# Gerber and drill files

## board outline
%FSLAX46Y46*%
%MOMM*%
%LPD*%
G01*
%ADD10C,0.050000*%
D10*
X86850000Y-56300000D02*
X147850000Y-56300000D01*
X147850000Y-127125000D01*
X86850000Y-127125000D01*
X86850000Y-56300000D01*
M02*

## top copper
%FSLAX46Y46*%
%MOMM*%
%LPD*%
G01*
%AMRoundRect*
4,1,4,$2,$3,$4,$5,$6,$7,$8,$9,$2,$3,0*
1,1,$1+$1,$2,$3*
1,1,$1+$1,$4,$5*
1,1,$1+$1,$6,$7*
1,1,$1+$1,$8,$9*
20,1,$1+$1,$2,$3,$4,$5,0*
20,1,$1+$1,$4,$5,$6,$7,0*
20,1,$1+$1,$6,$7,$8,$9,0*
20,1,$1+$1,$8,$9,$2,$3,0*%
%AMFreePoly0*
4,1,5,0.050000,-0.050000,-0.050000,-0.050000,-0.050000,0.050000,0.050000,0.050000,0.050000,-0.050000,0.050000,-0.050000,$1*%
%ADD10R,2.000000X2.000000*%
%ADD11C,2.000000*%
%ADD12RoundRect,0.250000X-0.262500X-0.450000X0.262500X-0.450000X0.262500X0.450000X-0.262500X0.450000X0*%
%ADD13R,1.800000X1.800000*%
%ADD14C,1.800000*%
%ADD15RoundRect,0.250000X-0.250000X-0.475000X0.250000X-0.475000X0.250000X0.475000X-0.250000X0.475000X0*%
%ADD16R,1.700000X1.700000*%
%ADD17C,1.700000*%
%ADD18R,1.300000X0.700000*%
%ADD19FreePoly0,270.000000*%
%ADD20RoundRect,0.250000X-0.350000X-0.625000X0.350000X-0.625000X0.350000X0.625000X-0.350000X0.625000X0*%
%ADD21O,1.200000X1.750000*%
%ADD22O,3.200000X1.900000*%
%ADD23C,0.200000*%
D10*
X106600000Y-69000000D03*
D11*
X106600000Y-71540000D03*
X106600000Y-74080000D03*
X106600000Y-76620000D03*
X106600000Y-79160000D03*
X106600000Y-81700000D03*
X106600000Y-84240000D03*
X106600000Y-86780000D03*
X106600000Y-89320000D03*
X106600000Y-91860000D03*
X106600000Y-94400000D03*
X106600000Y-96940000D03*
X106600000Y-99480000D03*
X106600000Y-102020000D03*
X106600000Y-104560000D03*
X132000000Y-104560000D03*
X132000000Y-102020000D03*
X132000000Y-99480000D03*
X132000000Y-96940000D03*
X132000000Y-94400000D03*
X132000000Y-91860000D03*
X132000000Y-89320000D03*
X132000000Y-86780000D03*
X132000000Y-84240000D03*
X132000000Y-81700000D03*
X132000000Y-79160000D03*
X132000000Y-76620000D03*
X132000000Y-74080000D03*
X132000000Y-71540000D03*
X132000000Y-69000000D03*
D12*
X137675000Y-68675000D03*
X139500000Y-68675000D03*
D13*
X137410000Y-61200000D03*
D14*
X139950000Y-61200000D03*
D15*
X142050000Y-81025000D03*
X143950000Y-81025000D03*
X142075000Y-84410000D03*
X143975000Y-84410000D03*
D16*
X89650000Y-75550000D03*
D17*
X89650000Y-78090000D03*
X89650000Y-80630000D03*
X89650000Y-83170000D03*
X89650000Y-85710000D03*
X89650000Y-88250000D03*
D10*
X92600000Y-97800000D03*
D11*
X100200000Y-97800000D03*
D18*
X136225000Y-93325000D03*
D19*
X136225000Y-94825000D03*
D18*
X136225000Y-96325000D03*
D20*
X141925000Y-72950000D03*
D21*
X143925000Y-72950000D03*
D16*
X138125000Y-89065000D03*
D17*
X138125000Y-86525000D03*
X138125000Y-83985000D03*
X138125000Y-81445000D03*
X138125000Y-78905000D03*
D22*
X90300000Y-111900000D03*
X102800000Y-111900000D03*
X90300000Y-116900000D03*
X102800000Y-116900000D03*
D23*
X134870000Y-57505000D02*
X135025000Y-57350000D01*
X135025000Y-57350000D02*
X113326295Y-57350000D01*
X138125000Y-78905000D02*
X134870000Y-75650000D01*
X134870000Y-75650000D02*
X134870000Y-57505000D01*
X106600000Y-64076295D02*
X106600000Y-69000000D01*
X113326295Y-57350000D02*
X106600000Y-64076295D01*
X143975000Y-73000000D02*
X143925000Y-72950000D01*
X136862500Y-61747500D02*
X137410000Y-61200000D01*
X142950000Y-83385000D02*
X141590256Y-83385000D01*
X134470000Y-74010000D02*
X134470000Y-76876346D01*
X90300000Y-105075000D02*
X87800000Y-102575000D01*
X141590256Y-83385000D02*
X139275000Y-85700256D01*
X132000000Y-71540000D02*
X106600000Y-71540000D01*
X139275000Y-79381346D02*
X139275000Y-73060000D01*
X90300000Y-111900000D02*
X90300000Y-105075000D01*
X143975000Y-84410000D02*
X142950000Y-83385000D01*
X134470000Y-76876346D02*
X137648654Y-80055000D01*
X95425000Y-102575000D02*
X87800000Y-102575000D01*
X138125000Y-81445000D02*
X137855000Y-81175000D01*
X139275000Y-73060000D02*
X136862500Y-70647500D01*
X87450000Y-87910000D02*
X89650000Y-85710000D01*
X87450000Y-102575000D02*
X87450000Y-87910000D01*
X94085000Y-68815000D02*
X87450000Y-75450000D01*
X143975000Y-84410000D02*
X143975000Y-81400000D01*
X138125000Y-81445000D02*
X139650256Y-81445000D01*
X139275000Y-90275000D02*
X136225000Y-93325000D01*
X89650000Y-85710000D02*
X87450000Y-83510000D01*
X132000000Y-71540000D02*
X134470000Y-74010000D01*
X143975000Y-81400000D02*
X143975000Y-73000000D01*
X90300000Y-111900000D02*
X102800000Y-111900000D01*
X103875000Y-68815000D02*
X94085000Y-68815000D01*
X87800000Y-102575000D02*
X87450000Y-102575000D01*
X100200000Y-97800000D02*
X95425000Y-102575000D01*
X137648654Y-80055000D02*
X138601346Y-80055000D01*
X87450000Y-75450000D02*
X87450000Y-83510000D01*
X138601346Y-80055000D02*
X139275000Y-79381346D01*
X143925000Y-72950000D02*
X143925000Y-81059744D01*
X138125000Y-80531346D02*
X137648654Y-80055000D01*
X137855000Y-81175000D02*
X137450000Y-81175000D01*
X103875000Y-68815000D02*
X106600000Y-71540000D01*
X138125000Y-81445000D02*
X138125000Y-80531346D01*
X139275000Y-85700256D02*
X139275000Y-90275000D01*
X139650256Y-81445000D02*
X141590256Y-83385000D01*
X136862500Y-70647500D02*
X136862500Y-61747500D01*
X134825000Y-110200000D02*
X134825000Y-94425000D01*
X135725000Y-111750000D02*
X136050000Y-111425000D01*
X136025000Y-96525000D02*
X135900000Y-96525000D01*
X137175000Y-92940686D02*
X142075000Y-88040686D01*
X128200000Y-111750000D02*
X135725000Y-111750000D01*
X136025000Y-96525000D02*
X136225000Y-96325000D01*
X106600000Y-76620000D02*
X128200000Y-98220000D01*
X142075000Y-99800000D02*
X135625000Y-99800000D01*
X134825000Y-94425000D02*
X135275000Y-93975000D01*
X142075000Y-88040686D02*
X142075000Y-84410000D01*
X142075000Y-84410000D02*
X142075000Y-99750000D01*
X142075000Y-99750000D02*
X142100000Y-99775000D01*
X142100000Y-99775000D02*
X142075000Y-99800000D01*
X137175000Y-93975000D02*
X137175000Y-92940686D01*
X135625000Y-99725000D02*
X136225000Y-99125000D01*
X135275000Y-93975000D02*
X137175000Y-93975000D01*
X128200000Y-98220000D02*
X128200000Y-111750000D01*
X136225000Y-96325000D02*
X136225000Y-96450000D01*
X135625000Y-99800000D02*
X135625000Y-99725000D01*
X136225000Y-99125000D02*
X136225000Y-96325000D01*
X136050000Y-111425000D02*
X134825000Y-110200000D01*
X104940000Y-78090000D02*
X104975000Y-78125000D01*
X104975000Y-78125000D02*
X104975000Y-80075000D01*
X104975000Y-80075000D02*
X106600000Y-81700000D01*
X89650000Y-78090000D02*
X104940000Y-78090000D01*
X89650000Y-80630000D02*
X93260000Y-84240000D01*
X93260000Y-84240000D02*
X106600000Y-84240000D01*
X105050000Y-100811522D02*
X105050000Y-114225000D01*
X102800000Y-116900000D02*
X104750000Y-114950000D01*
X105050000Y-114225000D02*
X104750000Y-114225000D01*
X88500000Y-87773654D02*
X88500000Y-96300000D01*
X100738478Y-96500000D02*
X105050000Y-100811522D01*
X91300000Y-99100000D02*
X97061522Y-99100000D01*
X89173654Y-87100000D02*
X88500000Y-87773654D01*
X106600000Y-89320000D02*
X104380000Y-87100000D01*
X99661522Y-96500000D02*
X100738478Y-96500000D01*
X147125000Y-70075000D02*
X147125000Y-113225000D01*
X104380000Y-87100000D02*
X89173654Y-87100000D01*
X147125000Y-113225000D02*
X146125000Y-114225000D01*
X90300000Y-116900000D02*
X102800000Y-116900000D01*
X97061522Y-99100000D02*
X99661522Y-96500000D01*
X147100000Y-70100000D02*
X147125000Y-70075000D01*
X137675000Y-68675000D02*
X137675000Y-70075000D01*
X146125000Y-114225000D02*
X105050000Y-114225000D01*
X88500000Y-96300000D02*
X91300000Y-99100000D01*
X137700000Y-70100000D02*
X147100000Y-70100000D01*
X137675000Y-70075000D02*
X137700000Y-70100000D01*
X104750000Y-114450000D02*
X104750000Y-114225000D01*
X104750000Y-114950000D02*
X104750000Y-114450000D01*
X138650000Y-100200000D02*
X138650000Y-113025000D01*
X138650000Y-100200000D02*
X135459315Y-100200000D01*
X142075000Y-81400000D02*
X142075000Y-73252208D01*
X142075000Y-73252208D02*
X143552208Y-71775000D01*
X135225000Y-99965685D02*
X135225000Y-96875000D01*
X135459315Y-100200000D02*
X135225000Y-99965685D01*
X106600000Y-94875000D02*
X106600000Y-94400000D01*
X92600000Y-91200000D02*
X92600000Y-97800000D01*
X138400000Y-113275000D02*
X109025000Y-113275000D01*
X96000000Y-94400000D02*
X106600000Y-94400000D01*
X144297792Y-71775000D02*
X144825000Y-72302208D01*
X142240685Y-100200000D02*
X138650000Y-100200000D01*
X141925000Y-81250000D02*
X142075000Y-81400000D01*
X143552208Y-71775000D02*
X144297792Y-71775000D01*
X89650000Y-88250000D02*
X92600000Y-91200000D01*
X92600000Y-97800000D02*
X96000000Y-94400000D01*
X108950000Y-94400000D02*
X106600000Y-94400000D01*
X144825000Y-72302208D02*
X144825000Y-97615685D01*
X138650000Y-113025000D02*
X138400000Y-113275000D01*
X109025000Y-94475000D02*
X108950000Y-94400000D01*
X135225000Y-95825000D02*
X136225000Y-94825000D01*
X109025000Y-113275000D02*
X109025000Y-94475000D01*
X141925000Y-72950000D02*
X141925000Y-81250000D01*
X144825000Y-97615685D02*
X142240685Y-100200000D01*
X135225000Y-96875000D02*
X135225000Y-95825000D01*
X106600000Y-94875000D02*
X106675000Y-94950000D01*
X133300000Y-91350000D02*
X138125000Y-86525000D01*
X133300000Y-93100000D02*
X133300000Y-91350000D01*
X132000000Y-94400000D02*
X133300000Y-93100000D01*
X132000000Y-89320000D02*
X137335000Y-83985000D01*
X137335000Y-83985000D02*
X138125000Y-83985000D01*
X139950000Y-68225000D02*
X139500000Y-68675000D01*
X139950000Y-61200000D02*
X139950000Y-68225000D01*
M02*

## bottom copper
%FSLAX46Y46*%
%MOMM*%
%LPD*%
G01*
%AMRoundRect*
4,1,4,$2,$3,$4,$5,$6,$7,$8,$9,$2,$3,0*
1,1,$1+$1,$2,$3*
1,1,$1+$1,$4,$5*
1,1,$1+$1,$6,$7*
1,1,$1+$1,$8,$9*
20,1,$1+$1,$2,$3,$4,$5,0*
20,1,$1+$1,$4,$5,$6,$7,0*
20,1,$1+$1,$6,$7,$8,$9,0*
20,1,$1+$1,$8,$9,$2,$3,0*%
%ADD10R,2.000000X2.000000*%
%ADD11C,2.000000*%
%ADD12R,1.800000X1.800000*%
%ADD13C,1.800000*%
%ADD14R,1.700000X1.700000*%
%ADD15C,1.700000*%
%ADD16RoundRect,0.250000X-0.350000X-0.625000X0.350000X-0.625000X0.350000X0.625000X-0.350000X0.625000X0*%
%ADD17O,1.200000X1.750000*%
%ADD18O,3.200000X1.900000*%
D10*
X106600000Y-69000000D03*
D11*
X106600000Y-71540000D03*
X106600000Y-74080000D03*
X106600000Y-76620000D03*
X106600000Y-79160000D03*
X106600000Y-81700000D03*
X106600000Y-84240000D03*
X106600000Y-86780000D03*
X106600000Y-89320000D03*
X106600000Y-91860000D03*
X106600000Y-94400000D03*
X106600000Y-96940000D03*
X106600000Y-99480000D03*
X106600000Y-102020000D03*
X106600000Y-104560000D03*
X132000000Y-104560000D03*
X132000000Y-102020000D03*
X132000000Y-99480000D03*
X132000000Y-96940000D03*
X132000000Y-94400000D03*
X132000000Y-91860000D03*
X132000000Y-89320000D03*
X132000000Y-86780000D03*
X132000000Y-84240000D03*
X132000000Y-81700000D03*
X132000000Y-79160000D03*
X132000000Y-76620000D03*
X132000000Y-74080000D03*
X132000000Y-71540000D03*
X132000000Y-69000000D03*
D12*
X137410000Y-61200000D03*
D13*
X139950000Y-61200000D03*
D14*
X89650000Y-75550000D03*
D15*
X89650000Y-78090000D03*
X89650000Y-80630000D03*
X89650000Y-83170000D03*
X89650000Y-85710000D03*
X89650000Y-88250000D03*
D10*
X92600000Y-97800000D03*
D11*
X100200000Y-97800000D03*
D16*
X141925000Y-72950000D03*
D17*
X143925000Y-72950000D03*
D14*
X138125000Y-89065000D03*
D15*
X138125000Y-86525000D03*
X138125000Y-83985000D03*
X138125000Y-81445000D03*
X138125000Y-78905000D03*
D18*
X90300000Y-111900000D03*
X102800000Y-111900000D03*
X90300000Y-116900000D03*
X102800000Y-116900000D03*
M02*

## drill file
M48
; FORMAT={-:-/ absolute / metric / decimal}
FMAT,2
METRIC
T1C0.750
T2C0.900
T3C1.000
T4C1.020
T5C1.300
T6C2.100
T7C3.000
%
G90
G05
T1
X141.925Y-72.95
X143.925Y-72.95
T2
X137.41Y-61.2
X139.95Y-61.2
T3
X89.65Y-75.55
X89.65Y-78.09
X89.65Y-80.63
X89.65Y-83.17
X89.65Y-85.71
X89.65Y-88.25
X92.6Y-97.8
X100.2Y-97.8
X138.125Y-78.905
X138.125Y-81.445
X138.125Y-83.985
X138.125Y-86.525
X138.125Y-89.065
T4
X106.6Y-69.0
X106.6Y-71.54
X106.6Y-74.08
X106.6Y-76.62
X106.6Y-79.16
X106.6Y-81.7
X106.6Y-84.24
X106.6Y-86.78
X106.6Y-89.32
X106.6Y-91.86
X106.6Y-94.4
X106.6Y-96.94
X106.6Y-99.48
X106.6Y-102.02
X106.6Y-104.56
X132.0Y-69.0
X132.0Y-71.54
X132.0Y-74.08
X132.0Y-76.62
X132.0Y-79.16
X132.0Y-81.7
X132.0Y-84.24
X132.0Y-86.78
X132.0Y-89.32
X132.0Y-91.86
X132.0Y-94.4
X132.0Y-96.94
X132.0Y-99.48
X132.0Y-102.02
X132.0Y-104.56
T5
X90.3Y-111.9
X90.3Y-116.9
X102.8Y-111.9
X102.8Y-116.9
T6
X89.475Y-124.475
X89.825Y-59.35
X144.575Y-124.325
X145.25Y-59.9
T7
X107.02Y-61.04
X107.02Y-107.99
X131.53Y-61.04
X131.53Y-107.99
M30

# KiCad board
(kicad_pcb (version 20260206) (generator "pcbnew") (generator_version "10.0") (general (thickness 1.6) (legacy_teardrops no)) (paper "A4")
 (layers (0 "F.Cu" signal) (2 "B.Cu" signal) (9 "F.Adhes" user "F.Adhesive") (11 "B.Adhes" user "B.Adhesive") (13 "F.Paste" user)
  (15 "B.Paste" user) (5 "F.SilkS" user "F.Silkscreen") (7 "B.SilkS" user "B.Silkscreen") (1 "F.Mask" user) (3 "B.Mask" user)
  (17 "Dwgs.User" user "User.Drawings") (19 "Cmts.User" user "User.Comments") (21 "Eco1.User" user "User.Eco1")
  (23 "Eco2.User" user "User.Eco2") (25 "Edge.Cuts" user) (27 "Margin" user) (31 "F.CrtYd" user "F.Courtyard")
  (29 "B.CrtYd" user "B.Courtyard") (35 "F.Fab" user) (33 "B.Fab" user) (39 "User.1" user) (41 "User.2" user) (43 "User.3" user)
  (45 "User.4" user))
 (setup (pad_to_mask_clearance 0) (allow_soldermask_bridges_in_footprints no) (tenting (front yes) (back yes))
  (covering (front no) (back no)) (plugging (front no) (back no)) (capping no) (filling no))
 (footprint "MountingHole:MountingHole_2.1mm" (layer "F.Cu") (at 89.475 124.475)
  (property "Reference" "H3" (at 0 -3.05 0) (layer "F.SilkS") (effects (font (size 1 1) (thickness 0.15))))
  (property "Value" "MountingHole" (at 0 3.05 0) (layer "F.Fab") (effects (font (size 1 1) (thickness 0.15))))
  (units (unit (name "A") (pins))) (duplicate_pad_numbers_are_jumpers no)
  (pad "" np_thru_hole circle (at 0 0) (size 2.1 2.1) (drill 2.1) (layers "*.Cu" "*.Mask")))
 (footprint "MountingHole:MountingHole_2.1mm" (layer "F.Cu") (at 145.25 59.9)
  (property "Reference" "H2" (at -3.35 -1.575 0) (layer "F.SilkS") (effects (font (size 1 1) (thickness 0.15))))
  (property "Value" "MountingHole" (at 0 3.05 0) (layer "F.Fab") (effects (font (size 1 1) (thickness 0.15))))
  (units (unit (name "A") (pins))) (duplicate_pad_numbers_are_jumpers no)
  (pad "" np_thru_hole circle (at 0 0) (size 2.1 2.1) (drill 2.1) (layers "*.Cu" "*.Mask")))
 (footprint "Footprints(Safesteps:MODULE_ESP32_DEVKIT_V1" (layer "F.Cu") (at 119.3 84.515)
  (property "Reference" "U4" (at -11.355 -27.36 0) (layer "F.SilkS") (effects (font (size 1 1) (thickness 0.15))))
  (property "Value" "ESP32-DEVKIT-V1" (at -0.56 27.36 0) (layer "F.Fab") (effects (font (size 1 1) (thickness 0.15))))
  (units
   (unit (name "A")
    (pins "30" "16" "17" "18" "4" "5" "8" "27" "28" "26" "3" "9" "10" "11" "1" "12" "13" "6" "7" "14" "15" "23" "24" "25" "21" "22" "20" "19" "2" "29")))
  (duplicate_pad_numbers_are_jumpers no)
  (pad "" np_thru_hole circle (at -12.28 -23.475) (size 3 3) (drill 3) (layers "*.Cu" "*.Mask"))
  (pad "" np_thru_hole circle (at -12.28 23.475) (size 3 3) (drill 3) (layers "*.Cu" "*.Mask"))
  (pad "" np_thru_hole circle (at 12.23 -23.475) (size 3 3) (drill 3) (layers "*.Cu" "*.Mask"))
  (pad "" np_thru_hole circle (at 12.23 23.475) (size 3 3) (drill 3) (layers "*.Cu" "*.Mask"))
  (pad "1" thru_hole rect (at -12.7 -15.515) (size 2 2) (drill 1.02) (layers "*.Cu" "*.Mask") (remove_unused_layers no) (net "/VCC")
   (solder_mask_margin 0.102))
  (pad "2" thru_hole circle (at -12.7 -12.975) (size 2 2) (drill 1.02) (layers "*.Cu" "*.Mask") (remove_unused_layers no) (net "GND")
   (solder_mask_margin 0.102))
  (pad "3" thru_hole circle (at -12.7 -10.435) (size 2 2) (drill 1.02) (layers "*.Cu" "*.Mask") (remove_unused_layers no)
   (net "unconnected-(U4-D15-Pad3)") (solder_mask_margin 0.102))
  (pad "4" thru_hole circle (at -12.7 -7.895) (size 2 2) (drill 1.02) (layers "*.Cu" "*.Mask") (remove_unused_layers no)
   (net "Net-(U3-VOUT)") (solder_mask_margin 0.102))
  (pad "5" thru_hole circle (at -12.7 -5.355) (size 2 2) (drill 1.02) (layers "*.Cu" "*.Mask") (remove_unused_layers no)
   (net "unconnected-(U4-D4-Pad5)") (solder_mask_margin 0.102))
  (pad "6" thru_hole circle (at -12.7 -2.815) (size 2 2) (drill 1.02) (layers "*.Cu" "*.Mask") (remove_unused_layers no) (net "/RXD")
   (solder_mask_margin 0.102))
  (pad "7" thru_hole circle (at -12.7 -0.275) (size 2 2) (drill 1.02) (layers "*.Cu" "*.Mask") (remove_unused_layers no) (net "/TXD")
   (solder_mask_margin 0.102))
  (pad "8" thru_hole circle (at -12.7 2.265) (size 2 2) (drill 1.02) (layers "*.Cu" "*.Mask") (remove_unused_layers no)
   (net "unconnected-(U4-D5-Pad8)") (solder_mask_margin 0.102))
  (pad "9" thru_hole circle (at -12.7 4.805) (size 2 2) (drill 1.02) (layers "*.Cu" "*.Mask") (remove_unused_layers no) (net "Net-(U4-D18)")
   (solder_mask_margin 0.102))
  (pad "10" thru_hole circle (at -12.7 7.345) (size 2 2) (drill 1.02) (layers "*.Cu" "*.Mask") (remove_unused_layers no)
   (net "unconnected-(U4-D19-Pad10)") (solder_mask_margin 0.102))
  (pad "11" thru_hole circle (at -12.7 9.885) (size 2 2) (drill 1.02) (layers "*.Cu" "*.Mask") (remove_unused_layers no) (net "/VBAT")
   (solder_mask_margin 0.102))
  (pad "12" thru_hole circle (at -12.7 12.425) (size 2 2) (drill 1.02) (layers "*.Cu" "*.Mask") (remove_unused_layers no)
   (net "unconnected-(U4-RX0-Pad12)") (solder_mask_margin 0.102))
  (pad "13" thru_hole circle (at -12.7 14.965) (size 2 2) (drill 1.02) (layers "*.Cu" "*.Mask") (remove_unused_layers no)
   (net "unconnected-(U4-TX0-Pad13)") (solder_mask_margin 0.102))
  (pad "14" thru_hole circle (at -12.7 17.505) (size 2 2) (drill 1.02) (layers "*.Cu" "*.Mask") (remove_unused_layers no)
   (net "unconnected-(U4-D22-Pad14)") (solder_mask_margin 0.102))
  (pad "15" thru_hole circle (at -12.7 20.045) (size 2 2) (drill 1.02) (layers "*.Cu" "*.Mask") (remove_unused_layers no)
   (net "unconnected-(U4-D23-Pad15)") (solder_mask_margin 0.102))
  (pad "16" thru_hole circle (at 12.7 20.045) (size 2 2) (drill 1.02) (layers "*.Cu" "*.Mask") (remove_unused_layers no)
   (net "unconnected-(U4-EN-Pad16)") (solder_mask_margin 0.102))
  (pad "17" thru_hole circle (at 12.7 17.505) (size 2 2) (drill 1.02) (layers "*.Cu" "*.Mask") (remove_unused_layers no)
   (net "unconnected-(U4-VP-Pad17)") (solder_mask_margin 0.102))
  (pad "18" thru_hole circle (at 12.7 14.965) (size 2 2) (drill 1.02) (layers "*.Cu" "*.Mask") (remove_unused_layers no)
   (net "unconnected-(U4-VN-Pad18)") (solder_mask_margin 0.102))
  (pad "19" thru_hole circle (at 12.7 12.425) (size 2 2) (drill 1.02) (layers "*.Cu" "*.Mask") (remove_unused_layers no)
   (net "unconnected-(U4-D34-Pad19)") (solder_mask_margin 0.102))
  (pad "20" thru_hole circle (at 12.7 9.885) (size 2 2) (drill 1.02) (layers "*.Cu" "*.Mask") (remove_unused_layers no) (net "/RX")
   (solder_mask_margin 0.102))
  (pad "21" thru_hole circle (at 12.7 7.345) (size 2 2) (drill 1.02) (layers "*.Cu" "*.Mask") (remove_unused_layers no)
   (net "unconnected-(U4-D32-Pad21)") (solder_mask_margin 0.102))
  (pad "22" thru_hole circle (at 12.7 4.805) (size 2 2) (drill 1.02) (layers "*.Cu" "*.Mask") (remove_unused_layers no) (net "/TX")
   (solder_mask_margin 0.102))
  (pad "23" thru_hole circle (at 12.7 2.265) (size 2 2) (drill 1.02) (layers "*.Cu" "*.Mask") (remove_unused_layers no)
   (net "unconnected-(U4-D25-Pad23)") (solder_mask_margin 0.102))
  (pad "24" thru_hole circle (at 12.7 -0.275) (size 2 2) (drill 1.02) (layers "*.Cu" "*.Mask") (remove_unused_layers no)
   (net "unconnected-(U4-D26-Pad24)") (solder_mask_margin 0.102))
  (pad "25" thru_hole circle (at 12.7 -2.815) (size 2 2) (drill 1.02) (layers "*.Cu" "*.Mask") (remove_unused_layers no)
   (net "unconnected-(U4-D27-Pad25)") (solder_mask_margin 0.102))
  (pad "26" thru_hole circle (at 12.7 -5.355) (size 2 2) (drill 1.02) (layers "*.Cu" "*.Mask") (remove_unused_layers no)
   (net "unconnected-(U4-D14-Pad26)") (solder_mask_margin 0.102))
  (pad "27" thru_hole circle (at 12.7 -7.895) (size 2 2) (drill 1.02) (layers "*.Cu" "*.Mask") (remove_unused_layers no)
   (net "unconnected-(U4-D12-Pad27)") (solder_mask_margin 0.102))
  (pad "28" thru_hole circle (at 12.7 -10.435) (size 2 2) (drill 1.02) (layers "*.Cu" "*.Mask") (remove_unused_layers no)
   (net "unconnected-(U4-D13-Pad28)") (solder_mask_margin 0.102))
  (pad "29" thru_hole circle (at 12.7 -12.975) (size 2 2) (drill 1.02) (layers "*.Cu" "*.Mask") (remove_unused_layers no) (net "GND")
   (solder_mask_margin 0.102))
  (pad "30" thru_hole circle (at 12.7 -15.515) (size 2 2) (drill 1.02) (layers "*.Cu" "*.Mask") (remove_unused_layers no)
   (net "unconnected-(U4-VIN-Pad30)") (solder_mask_margin 0.102))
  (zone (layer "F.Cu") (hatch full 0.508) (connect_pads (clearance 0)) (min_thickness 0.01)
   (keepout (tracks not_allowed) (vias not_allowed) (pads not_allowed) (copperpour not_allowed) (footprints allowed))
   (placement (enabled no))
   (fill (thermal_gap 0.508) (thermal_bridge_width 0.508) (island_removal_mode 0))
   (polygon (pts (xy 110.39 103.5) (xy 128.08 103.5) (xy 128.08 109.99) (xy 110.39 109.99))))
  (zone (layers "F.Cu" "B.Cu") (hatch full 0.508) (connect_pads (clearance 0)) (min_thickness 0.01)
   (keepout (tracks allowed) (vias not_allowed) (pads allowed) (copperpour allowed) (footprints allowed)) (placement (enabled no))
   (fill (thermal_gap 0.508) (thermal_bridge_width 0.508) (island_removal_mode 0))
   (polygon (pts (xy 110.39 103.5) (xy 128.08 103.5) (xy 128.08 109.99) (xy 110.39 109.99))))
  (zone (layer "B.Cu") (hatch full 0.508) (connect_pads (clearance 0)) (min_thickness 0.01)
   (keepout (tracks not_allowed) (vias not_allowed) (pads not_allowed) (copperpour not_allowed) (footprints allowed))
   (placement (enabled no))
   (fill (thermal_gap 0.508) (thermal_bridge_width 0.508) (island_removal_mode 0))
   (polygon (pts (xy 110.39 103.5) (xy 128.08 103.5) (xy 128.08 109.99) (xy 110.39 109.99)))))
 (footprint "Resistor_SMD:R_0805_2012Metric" (layer "F.Cu") (at 138.5875 68.675)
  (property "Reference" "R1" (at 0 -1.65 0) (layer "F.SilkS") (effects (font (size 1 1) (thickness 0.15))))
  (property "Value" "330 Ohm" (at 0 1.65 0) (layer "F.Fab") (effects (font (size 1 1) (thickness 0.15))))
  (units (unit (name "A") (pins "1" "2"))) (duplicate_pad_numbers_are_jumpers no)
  (pad "1" smd roundrect (at -0.9125 0) (size 1.025 1.4) (layers "F.Cu" "F.Mask" "F.Paste") (roundrect_rratio 0.243902) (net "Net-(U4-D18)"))
  (pad "2" smd roundrect (at 0.9125 0) (size 1.025 1.4) (layers "F.Cu" "F.Mask" "F.Paste") (roundrect_rratio 0.243902) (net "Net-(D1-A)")))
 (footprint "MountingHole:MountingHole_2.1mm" (layer "F.Cu") (at 144.575 124.325)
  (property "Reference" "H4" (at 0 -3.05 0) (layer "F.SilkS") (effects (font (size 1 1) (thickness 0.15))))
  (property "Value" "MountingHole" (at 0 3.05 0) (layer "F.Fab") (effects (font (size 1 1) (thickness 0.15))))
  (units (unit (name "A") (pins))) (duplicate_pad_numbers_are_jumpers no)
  (pad "" np_thru_hole circle (at 0 0) (size 2.1 2.1) (drill 2.1) (layers "*.Cu" "*.Mask")))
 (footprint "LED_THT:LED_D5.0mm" (layer "F.Cu") (at 137.41 61.2)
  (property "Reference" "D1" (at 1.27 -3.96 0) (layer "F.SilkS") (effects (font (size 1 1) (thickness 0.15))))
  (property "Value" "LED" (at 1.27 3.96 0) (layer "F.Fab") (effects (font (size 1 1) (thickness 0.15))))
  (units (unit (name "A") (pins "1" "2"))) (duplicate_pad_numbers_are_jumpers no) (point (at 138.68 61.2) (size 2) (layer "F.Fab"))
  (pad "1" thru_hole rect (at 0 0) (size 1.8 1.8) (drill 0.9) (layers "*.Cu" "*.Mask") (remove_unused_layers no) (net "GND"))
  (pad "2" thru_hole circle (at 2.54 0) (size 1.8 1.8) (drill 0.9) (layers "*.Cu" "*.Mask") (remove_unused_layers no) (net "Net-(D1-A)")))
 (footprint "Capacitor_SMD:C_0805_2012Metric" (layer "F.Cu") (at 143 81.025)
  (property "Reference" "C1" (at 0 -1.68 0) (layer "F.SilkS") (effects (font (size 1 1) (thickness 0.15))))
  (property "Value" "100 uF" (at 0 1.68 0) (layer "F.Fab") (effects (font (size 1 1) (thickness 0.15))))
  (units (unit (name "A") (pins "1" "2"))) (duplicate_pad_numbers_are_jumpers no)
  (pad "1" smd roundrect (at -0.95 0) (size 1 1.45) (layers "F.Cu" "F.Mask" "F.Paste") (roundrect_rratio 0.25) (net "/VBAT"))
  (pad "2" smd roundrect (at 0.95 0) (size 1 1.45) (layers "F.Cu" "F.Mask" "F.Paste") (roundrect_rratio 0.25) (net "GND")))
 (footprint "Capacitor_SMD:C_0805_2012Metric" (layer "F.Cu") (at 143.025 84.41)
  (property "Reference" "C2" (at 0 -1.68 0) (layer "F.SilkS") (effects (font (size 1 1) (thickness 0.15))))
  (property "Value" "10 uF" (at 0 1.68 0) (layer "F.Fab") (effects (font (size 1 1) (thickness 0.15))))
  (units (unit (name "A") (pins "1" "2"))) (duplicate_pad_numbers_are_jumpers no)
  (pad "1" smd roundrect (at -0.95 0) (size 1 1.45) (layers "F.Cu" "F.Mask" "F.Paste") (roundrect_rratio 0.25) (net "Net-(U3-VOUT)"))
  (pad "2" smd roundrect (at 0.95 0) (size 1 1.45) (layers "F.Cu" "F.Mask" "F.Paste") (roundrect_rratio 0.25) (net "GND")))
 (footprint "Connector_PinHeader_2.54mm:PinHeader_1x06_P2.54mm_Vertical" (layer "F.Cu") (at 89.65 75.55)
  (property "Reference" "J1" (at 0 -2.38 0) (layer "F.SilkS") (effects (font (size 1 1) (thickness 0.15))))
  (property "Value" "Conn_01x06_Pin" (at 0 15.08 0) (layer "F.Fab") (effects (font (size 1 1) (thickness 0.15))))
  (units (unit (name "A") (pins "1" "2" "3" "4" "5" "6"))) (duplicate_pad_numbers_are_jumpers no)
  (pad "1" thru_hole rect (at 0 0) (size 1.7 1.7) (drill 1) (layers "*.Cu" "*.Mask") (remove_unused_layers no) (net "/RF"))
  (pad "2" thru_hole circle (at 0 2.54) (size 1.7 1.7) (drill 1) (layers "*.Cu" "*.Mask") (remove_unused_layers no) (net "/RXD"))
  (pad "3" thru_hole circle (at 0 5.08) (size 1.7 1.7) (drill 1) (layers "*.Cu" "*.Mask") (remove_unused_layers no) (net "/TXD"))
  (pad "4" thru_hole circle (at 0 7.62) (size 1.7 1.7) (drill 1) (layers "*.Cu" "*.Mask") (remove_unused_layers no) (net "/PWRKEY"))
  (pad "5" thru_hole circle (at 0 10.16) (size 1.7 1.7) (drill 1) (layers "*.Cu" "*.Mask") (remove_unused_layers no) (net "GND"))
  (pad "6" thru_hole circle (at 0 12.7) (size 1.7 1.7) (drill 1) (layers "*.Cu" "*.Mask") (remove_unused_layers no) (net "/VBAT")))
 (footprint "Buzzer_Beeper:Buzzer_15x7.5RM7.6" (layer "F.Cu") (at 92.6 97.8)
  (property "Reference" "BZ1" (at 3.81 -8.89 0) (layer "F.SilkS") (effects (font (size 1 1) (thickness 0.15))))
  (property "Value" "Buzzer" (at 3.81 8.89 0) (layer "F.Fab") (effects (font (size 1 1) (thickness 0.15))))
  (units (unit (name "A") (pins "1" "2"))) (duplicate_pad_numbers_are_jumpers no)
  (pad "1" thru_hole rect (at 0 0) (size 2 2) (drill 1) (layers "*.Cu" "*.Mask") (remove_unused_layers no) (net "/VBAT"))
  (pad "2" thru_hole circle (at 7.6 0) (size 2 2) (drill 1) (layers "*.Cu" "*.Mask") (remove_unused_layers no) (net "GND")))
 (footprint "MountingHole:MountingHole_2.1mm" (layer "F.Cu") (at 89.825 59.35)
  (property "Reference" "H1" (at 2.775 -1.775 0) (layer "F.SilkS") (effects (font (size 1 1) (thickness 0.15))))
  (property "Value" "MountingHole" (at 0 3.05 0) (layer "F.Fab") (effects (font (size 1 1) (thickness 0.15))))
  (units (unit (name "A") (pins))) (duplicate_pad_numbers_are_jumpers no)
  (pad "" np_thru_hole circle (at 0 0) (size 2.1 2.1) (drill 2.1) (layers "*.Cu" "*.Mask")))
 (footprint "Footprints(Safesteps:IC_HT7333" (layer "F.Cu") (at 138.125 94.825 -90)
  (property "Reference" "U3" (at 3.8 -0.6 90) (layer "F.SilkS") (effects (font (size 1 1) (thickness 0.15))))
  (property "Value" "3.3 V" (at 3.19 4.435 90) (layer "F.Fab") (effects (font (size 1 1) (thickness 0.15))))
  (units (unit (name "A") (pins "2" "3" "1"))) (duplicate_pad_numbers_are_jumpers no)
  (pad "1" smd rect (at -1.5 1.9 270) (size 0.7 1.3) (layers "F.Cu" "F.Mask" "F.Paste") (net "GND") (solder_mask_margin 0.102))
  (pad "2" smd custom (at 0 1.9 270) (size 0.1 0.1) (layers "F.Cu") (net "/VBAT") (options (clearance outline) (anchor rect)) (primitives))
  (pad "3" smd rect (at 1.5 1.9 270) (size 0.7 1.3) (layers "F.Cu" "F.Mask" "F.Paste") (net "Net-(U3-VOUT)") (solder_mask_margin 0.102)))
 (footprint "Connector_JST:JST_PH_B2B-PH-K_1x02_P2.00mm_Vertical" (layer "F.Cu") (at 141.925 72.95)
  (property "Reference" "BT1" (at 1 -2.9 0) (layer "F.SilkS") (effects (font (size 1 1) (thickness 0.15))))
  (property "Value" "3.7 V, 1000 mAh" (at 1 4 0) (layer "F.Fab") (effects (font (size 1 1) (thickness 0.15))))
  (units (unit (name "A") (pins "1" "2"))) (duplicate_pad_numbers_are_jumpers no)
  (pad "1" thru_hole roundrect (at 0 0) (size 1.2 1.75) (drill 0.75) (layers "*.Cu" "*.Mask") (remove_unused_layers no)
   (roundrect_rratio 0.208333) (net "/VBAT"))
  (pad "2" thru_hole oval (at 2 0) (size 1.2 1.75) (drill 0.75) (layers "*.Cu" "*.Mask") (remove_unused_layers no) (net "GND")))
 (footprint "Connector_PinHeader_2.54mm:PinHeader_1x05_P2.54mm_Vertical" (layer "F.Cu") (at 138.125 89.065 180)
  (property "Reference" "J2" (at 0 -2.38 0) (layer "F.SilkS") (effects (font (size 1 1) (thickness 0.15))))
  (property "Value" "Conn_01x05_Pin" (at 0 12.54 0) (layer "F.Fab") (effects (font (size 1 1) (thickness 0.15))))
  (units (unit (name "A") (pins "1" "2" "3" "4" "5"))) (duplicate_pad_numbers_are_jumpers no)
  (pad "1" thru_hole rect (at 0 0 180) (size 1.7 1.7) (drill 1) (layers "*.Cu" "*.Mask") (remove_unused_layers no) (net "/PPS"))
  (pad "2" thru_hole circle (at 0 2.54 180) (size 1.7 1.7) (drill 1) (layers "*.Cu" "*.Mask") (remove_unused_layers no) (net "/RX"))
  (pad "3" thru_hole circle (at 0 5.08 180) (size 1.7 1.7) (drill 1) (layers "*.Cu" "*.Mask") (remove_unused_layers no) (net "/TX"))
  (pad "4" thru_hole circle (at 0 7.62 180) (size 1.7 1.7) (drill 1) (layers "*.Cu" "*.Mask") (remove_unused_layers no) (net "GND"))
  (pad "5" thru_hole circle (at 0 10.16 180) (size 1.7 1.7) (drill 1) (layers "*.Cu" "*.Mask") (remove_unused_layers no) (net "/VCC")))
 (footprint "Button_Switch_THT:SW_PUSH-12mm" (layer "F.Cu") (at 90.3 111.9)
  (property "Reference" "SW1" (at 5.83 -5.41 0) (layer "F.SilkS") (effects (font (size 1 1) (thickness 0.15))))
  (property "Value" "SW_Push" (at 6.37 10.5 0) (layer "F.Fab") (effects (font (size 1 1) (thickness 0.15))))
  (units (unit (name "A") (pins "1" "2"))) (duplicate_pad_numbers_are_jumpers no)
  (pad "1" thru_hole oval (at 0 0) (size 3.2 1.9) (drill 1.3) (layers "*.Cu" "*.Mask") (remove_unused_layers no) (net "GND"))
  (pad "1" thru_hole oval (at 12.5 0) (size 3.2 1.9) (drill 1.3) (layers "*.Cu" "*.Mask") (remove_unused_layers no) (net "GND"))
  (pad "2" thru_hole oval (at 0 5) (size 3.2 1.9) (drill 1.3) (layers "*.Cu" "*.Mask") (remove_unused_layers no) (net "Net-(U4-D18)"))
  (pad "2" thru_hole oval (at 12.5 5) (size 3.2 1.9) (drill 1.3) (layers "*.Cu" "*.Mask") (remove_unused_layers no) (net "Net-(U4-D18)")))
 (gr_rect (start 86.85 56.3) (end 147.85 127.125) (stroke (width 0.05) (type default)) (fill no) (layer "Edge.Cuts"))
 (segment (start 134.87 57.505) (end 135.025 57.35) (width 0.2) (layer "F.Cu") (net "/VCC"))
 (segment (start 135.025 57.35) (end 113.326295 57.35) (width 0.2) (layer "F.Cu") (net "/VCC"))
 (segment (start 138.125 78.905) (end 134.87 75.65) (width 0.2) (layer "F.Cu") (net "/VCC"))
 (segment (start 134.87 75.65) (end 134.87 57.505) (width 0.2) (layer "F.Cu") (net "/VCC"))
 (segment (start 106.6 64.076295) (end 106.6 69) (width 0.2) (layer "F.Cu") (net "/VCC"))
 (segment (start 113.326295 57.35) (end 106.6 64.076295) (width 0.2) (layer "F.Cu") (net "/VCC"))
 (segment (start 143.975 73) (end 143.925 72.95) (width 0.2) (layer "F.Cu") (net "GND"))
 (segment (start 136.8625 61.7475) (end 137.41 61.2) (width 0.2) (layer "F.Cu") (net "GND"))
 (segment (start 142.95 83.385) (end 141.590256 83.385) (width 0.2) (layer "F.Cu") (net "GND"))
 (segment (start 134.47 74.01) (end 134.47 76.876346) (width 0.2) (layer "F.Cu") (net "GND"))
 (segment (start 90.3 105.075) (end 87.8 102.575) (width 0.2) (layer "F.Cu") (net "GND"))
 (segment (start 141.590256 83.385) (end 139.275 85.700256) (width 0.2) (layer "F.Cu") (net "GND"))
 (segment (start 132 71.54) (end 106.6 71.54) (width 0.2) (layer "F.Cu") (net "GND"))
 (segment (start 139.275 79.381346) (end 139.275 73.06) (width 0.2) (layer "F.Cu") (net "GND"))
 (segment (start 90.3 111.9) (end 90.3 105.075) (width 0.2) (layer "F.Cu") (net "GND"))
 (segment (start 143.975 84.41) (end 142.95 83.385) (width 0.2) (layer "F.Cu") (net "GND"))
 (segment (start 134.47 76.876346) (end 137.648654 80.055) (width 0.2) (layer "F.Cu") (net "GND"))
 (segment (start 95.425 102.575) (end 87.8 102.575) (width 0.2) (layer "F.Cu") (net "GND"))
 (segment (start 138.125 81.445) (end 137.855 81.175) (width 0.2) (layer "F.Cu") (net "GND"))
 (segment (start 139.275 73.06) (end 136.8625 70.6475) (width 0.2) (layer "F.Cu") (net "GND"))
 (segment (start 87.45 87.91) (end 89.65 85.71) (width 0.2) (layer "F.Cu") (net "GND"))
 (segment (start 87.45 102.575) (end 87.45 87.91) (width 0.2) (layer "F.Cu") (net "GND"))
 (segment (start 94.085 68.815) (end 87.45 75.45) (width 0.2) (layer "F.Cu") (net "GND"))
 (segment (start 143.975 84.41) (end 143.975 81.4) (width 0.2) (layer "F.Cu") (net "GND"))
 (segment (start 138.125 81.445) (end 139.650256 81.445) (width 0.2) (layer "F.Cu") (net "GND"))
 (segment (start 139.275 90.275) (end 136.225 93.325) (width 0.2) (layer "F.Cu") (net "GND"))
 (segment (start 89.65 85.71) (end 87.45 83.51) (width 0.2) (layer "F.Cu") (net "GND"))
 (segment (start 132 71.54) (end 134.47 74.01) (width 0.2) (layer "F.Cu") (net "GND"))
 (segment (start 143.975 81.4) (end 143.975 73) (width 0.2) (layer "F.Cu") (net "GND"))
 (segment (start 90.3 111.9) (end 102.8 111.9) (width 0.2) (layer "F.Cu") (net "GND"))
 (segment (start 103.875 68.815) (end 94.085 68.815) (width 0.2) (layer "F.Cu") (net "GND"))
 (segment (start 87.8 102.575) (end 87.45 102.575) (width 0.2) (layer "F.Cu") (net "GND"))
 (segment (start 100.2 97.8) (end 95.425 102.575) (width 0.2) (layer "F.Cu") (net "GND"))
 (segment (start 137.648654 80.055) (end 138.601346 80.055) (width 0.2) (layer "F.Cu") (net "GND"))
 (segment (start 87.45 75.45) (end 87.45 83.51) (width 0.2) (layer "F.Cu") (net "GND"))
 (segment (start 138.601346 80.055) (end 139.275 79.381346) (width 0.2) (layer "F.Cu") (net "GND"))
 (segment (start 143.925 72.95) (end 143.925 81.059744) (width 0.2) (layer "F.Cu") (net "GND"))
 (segment (start 138.125 80.531346) (end 137.648654 80.055) (width 0.2) (layer "F.Cu") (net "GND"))
 (segment (start 137.855 81.175) (end 137.45 81.175) (width 0.2) (layer "F.Cu") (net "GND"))
 (segment (start 103.875 68.815) (end 106.6 71.54) (width 0.2) (layer "F.Cu") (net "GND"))
 (segment (start 138.125 81.445) (end 138.125 80.531346) (width 0.2) (layer "F.Cu") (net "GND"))
 (segment (start 139.275 85.700256) (end 139.275 90.275) (width 0.2) (layer "F.Cu") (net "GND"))
 (segment (start 139.650256 81.445) (end 141.590256 83.385) (width 0.2) (layer "F.Cu") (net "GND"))
 (segment (start 136.8625 70.6475) (end 136.8625 61.7475) (width 0.2) (layer "F.Cu") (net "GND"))
 (segment (start 134.825 110.2) (end 134.825 94.425) (width 0.2) (layer "F.Cu") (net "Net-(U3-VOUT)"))
 (segment (start 135.725 111.75) (end 136.05 111.425) (width 0.2) (layer "F.Cu") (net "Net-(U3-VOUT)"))
 (segment (start 136.025 96.525) (end 135.9 96.525) (width 0.2) (layer "F.Cu") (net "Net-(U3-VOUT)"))
 (segment (start 137.175 92.940686) (end 142.075 88.040686) (width 0.2) (layer "F.Cu") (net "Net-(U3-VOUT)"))
 (segment (start 128.2 111.75) (end 135.725 111.75) (width 0.2) (layer "F.Cu") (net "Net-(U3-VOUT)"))
 (segment (start 136.025 96.525) (end 136.225 96.325) (width 0.2) (layer "F.Cu") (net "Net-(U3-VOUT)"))
 (segment (start 106.6 76.62) (end 128.2 98.22) (width 0.2) (layer "F.Cu") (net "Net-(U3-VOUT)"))
 (segment (start 142.075 99.8) (end 135.625 99.8) (width 0.2) (layer "F.Cu") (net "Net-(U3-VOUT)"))
 (segment (start 134.825 94.425) (end 135.275 93.975) (width 0.2) (layer "F.Cu") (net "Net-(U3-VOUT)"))
 (segment (start 142.075 88.040686) (end 142.075 84.41) (width 0.2) (layer "F.Cu") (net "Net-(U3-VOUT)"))
 (segment (start 142.075 84.41) (end 142.075 99.75) (width 0.2) (layer "F.Cu") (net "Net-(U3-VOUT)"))
 (segment (start 142.075 99.75) (end 142.1 99.775) (width 0.2) (layer "F.Cu") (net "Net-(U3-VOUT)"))
 (segment (start 142.1 99.775) (end 142.075 99.8) (width 0.2) (layer "F.Cu") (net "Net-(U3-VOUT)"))
 (segment (start 137.175 93.975) (end 137.175 92.940686) (width 0.2) (layer "F.Cu") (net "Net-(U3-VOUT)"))
 (segment (start 135.625 99.725) (end 136.225 99.125) (width 0.2) (layer "F.Cu") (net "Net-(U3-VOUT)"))
 (segment (start 135.275 93.975) (end 137.175 93.975) (width 0.2) (layer "F.Cu") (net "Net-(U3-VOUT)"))
 (segment (start 128.2 98.22) (end 128.2 111.75) (width 0.2) (layer "F.Cu") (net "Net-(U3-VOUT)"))
 (segment (start 136.225 96.325) (end 136.225 96.45) (width 0.2) (layer "F.Cu") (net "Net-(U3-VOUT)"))
 (segment (start 135.625 99.8) (end 135.625 99.725) (width 0.2) (layer "F.Cu") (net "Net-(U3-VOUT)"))
 (segment (start 136.225 99.125) (end 136.225 96.325) (width 0.2) (layer "F.Cu") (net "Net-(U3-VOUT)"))
 (segment (start 136.05 111.425) (end 134.825 110.2) (width 0.2) (layer "F.Cu") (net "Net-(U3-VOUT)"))
 (segment (start 104.94 78.09) (end 104.975 78.125) (width 0.2) (layer "F.Cu") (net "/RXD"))
 (segment (start 104.975 78.125) (end 104.975 80.075) (width 0.2) (layer "F.Cu") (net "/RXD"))
 (segment (start 104.975 80.075) (end 106.6 81.7) (width 0.2) (layer "F.Cu") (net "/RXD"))
 (segment (start 89.65 78.09) (end 104.94 78.09) (width 0.2) (layer "F.Cu") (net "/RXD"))
 (segment (start 89.65 80.63) (end 93.26 84.24) (width 0.2) (layer "F.Cu") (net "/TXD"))
 (segment (start 93.26 84.24) (end 106.6 84.24) (width 0.2) (layer "F.Cu") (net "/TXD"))
 (segment (start 105.05 100.811522) (end 105.05 114.225) (width 0.2) (layer "F.Cu") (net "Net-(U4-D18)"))
 (segment (start 102.8 116.9) (end 104.75 114.95) (width 0.2) (layer "F.Cu") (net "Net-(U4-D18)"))
 (segment (start 105.05 114.225) (end 104.75 114.225) (width 0.2) (layer "F.Cu") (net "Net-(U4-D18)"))
 (segment (start 88.5 87.773654) (end 88.5 96.3) (width 0.2) (layer "F.Cu") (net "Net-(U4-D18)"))
 (segment (start 100.738478 96.5) (end 105.05 100.811522) (width 0.2) (layer "F.Cu") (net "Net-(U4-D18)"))
 (segment (start 91.3 99.1) (end 97.061522 99.1) (width 0.2) (layer "F.Cu") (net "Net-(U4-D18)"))
 (segment (start 89.173654 87.1) (end 88.5 87.773654) (width 0.2) (layer "F.Cu") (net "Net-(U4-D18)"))
 (segment (start 106.6 89.32) (end 104.38 87.1) (width 0.2) (layer "F.Cu") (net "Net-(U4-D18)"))
 (segment (start 99.661522 96.5) (end 100.738478 96.5) (width 0.2) (layer "F.Cu") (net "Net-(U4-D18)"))
 (segment (start 147.125 70.075) (end 147.125 113.225) (width 0.2) (layer "F.Cu") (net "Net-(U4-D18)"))
 (segment (start 104.38 87.1) (end 89.173654 87.1) (width 0.2) (layer "F.Cu") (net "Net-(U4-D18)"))
 (segment (start 147.125 113.225) (end 146.125 114.225) (width 0.2) (layer "F.Cu") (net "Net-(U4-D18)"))
 (segment (start 90.3 116.9) (end 102.8 116.9) (width 0.2) (layer "F.Cu") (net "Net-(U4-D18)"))
 (segment (start 97.061522 99.1) (end 99.661522 96.5) (width 0.2) (layer "F.Cu") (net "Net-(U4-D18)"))
 (segment (start 147.1 70.1) (end 147.125 70.075) (width 0.2) (layer "F.Cu") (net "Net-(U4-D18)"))
 (segment (start 137.675 68.675) (end 137.675 70.075) (width 0.2) (layer "F.Cu") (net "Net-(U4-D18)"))
 (segment (start 146.125 114.225) (end 105.05 114.225) (width 0.2) (layer "F.Cu") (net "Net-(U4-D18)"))
 (segment (start 88.5 96.3) (end 91.3 99.1) (width 0.2) (layer "F.Cu") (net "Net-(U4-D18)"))
 (segment (start 137.7 70.1) (end 147.1 70.1) (width 0.2) (layer "F.Cu") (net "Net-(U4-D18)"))
 (segment (start 137.675 70.075) (end 137.7 70.1) (width 0.2) (layer "F.Cu") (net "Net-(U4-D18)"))
 (segment (start 104.75 114.45) (end 104.75 114.225) (width 0.2) (layer "F.Cu") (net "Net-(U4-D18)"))
 (segment (start 104.75 114.95) (end 104.75 114.45) (width 0.2) (layer "F.Cu") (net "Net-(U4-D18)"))
 (segment (start 138.65 100.2) (end 138.65 113.025) (width 0.2) (layer "F.Cu") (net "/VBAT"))
 (segment (start 138.65 100.2) (end 135.459315 100.2) (width 0.2) (layer "F.Cu") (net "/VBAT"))
 (segment (start 142.075 81.4) (end 142.075 73.252208) (width 0.2) (layer "F.Cu") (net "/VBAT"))
 (segment (start 142.075 73.252208) (end 143.552208 71.775) (width 0.2) (layer "F.Cu") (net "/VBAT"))
 (segment (start 135.225 99.965685) (end 135.225 96.875) (width 0.2) (layer "F.Cu") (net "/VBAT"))
 (segment (start 135.459315 100.2) (end 135.225 99.965685) (width 0.2) (layer "F.Cu") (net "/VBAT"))
 (segment (start 106.6 94.875) (end 106.6 94.4) (width 0.2) (layer "F.Cu") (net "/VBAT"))
 (segment (start 92.6 91.2) (end 92.6 97.8) (width 0.2) (layer "F.Cu") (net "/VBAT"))
 (segment (start 138.4 113.275) (end 109.025 113.275) (width 0.2) (layer "F.Cu") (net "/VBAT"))
 (segment (start 96 94.4) (end 106.6 94.4) (width 0.2) (layer "F.Cu") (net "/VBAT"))
 (segment (start 144.297792 71.775) (end 144.825 72.302208) (width 0.2) (layer "F.Cu") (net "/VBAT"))
 (segment (start 142.240685 100.2) (end 138.65 100.2) (width 0.2) (layer "F.Cu") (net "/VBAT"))
 (segment (start 141.925 81.25) (end 142.075 81.4) (width 0.2) (layer "F.Cu") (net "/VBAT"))
 (segment (start 143.552208 71.775) (end 144.297792 71.775) (width 0.2) (layer "F.Cu") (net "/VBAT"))
 (segment (start 89.65 88.25) (end 92.6 91.2) (width 0.2) (layer "F.Cu") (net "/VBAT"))
 (segment (start 92.6 97.8) (end 96 94.4) (width 0.2) (layer "F.Cu") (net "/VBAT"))
 (segment (start 108.95 94.4) (end 106.6 94.4) (width 0.2) (layer "F.Cu") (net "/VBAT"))
 (segment (start 144.825 72.302208) (end 144.825 97.615685) (width 0.2) (layer "F.Cu") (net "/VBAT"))
 (segment (start 138.65 113.025) (end 138.4 113.275) (width 0.2) (layer "F.Cu") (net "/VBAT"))
 (segment (start 109.025 94.475) (end 108.95 94.4) (width 0.2) (layer "F.Cu") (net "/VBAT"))
 (segment (start 135.225 95.825) (end 136.225 94.825) (width 0.2) (layer "F.Cu") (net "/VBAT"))
 (segment (start 109.025 113.275) (end 109.025 94.475) (width 0.2) (layer "F.Cu") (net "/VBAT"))
 (segment (start 141.925 72.95) (end 141.925 81.25) (width 0.2) (layer "F.Cu") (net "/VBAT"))
 (segment (start 144.825 97.615685) (end 142.240685 100.2) (width 0.2) (layer "F.Cu") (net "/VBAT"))
 (segment (start 135.225 96.875) (end 135.225 95.825) (width 0.2) (layer "F.Cu") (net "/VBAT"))
 (segment (start 106.6 94.875) (end 106.675 94.95) (width 0.2) (layer "F.Cu") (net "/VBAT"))
 (segment (start 133.3 91.35) (end 138.125 86.525) (width 0.2) (layer "F.Cu") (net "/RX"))
 (segment (start 133.3 93.1) (end 133.3 91.35) (width 0.2) (layer "F.Cu") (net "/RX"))
 (segment (start 132 94.4) (end 133.3 93.1) (width 0.2) (layer "F.Cu") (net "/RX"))
 (segment (start 132 89.32) (end 137.335 83.985) (width 0.2) (layer "F.Cu") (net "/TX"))
 (segment (start 137.335 83.985) (end 138.125 83.985) (width 0.2) (layer "F.Cu") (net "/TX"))
 (segment (start 139.95 68.225) (end 139.5 68.675) (width 0.2) (layer "F.Cu") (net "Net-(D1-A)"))
 (segment (start 139.95 61.2) (end 139.95 68.225) (width 0.2) (layer "F.Cu") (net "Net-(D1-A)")))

